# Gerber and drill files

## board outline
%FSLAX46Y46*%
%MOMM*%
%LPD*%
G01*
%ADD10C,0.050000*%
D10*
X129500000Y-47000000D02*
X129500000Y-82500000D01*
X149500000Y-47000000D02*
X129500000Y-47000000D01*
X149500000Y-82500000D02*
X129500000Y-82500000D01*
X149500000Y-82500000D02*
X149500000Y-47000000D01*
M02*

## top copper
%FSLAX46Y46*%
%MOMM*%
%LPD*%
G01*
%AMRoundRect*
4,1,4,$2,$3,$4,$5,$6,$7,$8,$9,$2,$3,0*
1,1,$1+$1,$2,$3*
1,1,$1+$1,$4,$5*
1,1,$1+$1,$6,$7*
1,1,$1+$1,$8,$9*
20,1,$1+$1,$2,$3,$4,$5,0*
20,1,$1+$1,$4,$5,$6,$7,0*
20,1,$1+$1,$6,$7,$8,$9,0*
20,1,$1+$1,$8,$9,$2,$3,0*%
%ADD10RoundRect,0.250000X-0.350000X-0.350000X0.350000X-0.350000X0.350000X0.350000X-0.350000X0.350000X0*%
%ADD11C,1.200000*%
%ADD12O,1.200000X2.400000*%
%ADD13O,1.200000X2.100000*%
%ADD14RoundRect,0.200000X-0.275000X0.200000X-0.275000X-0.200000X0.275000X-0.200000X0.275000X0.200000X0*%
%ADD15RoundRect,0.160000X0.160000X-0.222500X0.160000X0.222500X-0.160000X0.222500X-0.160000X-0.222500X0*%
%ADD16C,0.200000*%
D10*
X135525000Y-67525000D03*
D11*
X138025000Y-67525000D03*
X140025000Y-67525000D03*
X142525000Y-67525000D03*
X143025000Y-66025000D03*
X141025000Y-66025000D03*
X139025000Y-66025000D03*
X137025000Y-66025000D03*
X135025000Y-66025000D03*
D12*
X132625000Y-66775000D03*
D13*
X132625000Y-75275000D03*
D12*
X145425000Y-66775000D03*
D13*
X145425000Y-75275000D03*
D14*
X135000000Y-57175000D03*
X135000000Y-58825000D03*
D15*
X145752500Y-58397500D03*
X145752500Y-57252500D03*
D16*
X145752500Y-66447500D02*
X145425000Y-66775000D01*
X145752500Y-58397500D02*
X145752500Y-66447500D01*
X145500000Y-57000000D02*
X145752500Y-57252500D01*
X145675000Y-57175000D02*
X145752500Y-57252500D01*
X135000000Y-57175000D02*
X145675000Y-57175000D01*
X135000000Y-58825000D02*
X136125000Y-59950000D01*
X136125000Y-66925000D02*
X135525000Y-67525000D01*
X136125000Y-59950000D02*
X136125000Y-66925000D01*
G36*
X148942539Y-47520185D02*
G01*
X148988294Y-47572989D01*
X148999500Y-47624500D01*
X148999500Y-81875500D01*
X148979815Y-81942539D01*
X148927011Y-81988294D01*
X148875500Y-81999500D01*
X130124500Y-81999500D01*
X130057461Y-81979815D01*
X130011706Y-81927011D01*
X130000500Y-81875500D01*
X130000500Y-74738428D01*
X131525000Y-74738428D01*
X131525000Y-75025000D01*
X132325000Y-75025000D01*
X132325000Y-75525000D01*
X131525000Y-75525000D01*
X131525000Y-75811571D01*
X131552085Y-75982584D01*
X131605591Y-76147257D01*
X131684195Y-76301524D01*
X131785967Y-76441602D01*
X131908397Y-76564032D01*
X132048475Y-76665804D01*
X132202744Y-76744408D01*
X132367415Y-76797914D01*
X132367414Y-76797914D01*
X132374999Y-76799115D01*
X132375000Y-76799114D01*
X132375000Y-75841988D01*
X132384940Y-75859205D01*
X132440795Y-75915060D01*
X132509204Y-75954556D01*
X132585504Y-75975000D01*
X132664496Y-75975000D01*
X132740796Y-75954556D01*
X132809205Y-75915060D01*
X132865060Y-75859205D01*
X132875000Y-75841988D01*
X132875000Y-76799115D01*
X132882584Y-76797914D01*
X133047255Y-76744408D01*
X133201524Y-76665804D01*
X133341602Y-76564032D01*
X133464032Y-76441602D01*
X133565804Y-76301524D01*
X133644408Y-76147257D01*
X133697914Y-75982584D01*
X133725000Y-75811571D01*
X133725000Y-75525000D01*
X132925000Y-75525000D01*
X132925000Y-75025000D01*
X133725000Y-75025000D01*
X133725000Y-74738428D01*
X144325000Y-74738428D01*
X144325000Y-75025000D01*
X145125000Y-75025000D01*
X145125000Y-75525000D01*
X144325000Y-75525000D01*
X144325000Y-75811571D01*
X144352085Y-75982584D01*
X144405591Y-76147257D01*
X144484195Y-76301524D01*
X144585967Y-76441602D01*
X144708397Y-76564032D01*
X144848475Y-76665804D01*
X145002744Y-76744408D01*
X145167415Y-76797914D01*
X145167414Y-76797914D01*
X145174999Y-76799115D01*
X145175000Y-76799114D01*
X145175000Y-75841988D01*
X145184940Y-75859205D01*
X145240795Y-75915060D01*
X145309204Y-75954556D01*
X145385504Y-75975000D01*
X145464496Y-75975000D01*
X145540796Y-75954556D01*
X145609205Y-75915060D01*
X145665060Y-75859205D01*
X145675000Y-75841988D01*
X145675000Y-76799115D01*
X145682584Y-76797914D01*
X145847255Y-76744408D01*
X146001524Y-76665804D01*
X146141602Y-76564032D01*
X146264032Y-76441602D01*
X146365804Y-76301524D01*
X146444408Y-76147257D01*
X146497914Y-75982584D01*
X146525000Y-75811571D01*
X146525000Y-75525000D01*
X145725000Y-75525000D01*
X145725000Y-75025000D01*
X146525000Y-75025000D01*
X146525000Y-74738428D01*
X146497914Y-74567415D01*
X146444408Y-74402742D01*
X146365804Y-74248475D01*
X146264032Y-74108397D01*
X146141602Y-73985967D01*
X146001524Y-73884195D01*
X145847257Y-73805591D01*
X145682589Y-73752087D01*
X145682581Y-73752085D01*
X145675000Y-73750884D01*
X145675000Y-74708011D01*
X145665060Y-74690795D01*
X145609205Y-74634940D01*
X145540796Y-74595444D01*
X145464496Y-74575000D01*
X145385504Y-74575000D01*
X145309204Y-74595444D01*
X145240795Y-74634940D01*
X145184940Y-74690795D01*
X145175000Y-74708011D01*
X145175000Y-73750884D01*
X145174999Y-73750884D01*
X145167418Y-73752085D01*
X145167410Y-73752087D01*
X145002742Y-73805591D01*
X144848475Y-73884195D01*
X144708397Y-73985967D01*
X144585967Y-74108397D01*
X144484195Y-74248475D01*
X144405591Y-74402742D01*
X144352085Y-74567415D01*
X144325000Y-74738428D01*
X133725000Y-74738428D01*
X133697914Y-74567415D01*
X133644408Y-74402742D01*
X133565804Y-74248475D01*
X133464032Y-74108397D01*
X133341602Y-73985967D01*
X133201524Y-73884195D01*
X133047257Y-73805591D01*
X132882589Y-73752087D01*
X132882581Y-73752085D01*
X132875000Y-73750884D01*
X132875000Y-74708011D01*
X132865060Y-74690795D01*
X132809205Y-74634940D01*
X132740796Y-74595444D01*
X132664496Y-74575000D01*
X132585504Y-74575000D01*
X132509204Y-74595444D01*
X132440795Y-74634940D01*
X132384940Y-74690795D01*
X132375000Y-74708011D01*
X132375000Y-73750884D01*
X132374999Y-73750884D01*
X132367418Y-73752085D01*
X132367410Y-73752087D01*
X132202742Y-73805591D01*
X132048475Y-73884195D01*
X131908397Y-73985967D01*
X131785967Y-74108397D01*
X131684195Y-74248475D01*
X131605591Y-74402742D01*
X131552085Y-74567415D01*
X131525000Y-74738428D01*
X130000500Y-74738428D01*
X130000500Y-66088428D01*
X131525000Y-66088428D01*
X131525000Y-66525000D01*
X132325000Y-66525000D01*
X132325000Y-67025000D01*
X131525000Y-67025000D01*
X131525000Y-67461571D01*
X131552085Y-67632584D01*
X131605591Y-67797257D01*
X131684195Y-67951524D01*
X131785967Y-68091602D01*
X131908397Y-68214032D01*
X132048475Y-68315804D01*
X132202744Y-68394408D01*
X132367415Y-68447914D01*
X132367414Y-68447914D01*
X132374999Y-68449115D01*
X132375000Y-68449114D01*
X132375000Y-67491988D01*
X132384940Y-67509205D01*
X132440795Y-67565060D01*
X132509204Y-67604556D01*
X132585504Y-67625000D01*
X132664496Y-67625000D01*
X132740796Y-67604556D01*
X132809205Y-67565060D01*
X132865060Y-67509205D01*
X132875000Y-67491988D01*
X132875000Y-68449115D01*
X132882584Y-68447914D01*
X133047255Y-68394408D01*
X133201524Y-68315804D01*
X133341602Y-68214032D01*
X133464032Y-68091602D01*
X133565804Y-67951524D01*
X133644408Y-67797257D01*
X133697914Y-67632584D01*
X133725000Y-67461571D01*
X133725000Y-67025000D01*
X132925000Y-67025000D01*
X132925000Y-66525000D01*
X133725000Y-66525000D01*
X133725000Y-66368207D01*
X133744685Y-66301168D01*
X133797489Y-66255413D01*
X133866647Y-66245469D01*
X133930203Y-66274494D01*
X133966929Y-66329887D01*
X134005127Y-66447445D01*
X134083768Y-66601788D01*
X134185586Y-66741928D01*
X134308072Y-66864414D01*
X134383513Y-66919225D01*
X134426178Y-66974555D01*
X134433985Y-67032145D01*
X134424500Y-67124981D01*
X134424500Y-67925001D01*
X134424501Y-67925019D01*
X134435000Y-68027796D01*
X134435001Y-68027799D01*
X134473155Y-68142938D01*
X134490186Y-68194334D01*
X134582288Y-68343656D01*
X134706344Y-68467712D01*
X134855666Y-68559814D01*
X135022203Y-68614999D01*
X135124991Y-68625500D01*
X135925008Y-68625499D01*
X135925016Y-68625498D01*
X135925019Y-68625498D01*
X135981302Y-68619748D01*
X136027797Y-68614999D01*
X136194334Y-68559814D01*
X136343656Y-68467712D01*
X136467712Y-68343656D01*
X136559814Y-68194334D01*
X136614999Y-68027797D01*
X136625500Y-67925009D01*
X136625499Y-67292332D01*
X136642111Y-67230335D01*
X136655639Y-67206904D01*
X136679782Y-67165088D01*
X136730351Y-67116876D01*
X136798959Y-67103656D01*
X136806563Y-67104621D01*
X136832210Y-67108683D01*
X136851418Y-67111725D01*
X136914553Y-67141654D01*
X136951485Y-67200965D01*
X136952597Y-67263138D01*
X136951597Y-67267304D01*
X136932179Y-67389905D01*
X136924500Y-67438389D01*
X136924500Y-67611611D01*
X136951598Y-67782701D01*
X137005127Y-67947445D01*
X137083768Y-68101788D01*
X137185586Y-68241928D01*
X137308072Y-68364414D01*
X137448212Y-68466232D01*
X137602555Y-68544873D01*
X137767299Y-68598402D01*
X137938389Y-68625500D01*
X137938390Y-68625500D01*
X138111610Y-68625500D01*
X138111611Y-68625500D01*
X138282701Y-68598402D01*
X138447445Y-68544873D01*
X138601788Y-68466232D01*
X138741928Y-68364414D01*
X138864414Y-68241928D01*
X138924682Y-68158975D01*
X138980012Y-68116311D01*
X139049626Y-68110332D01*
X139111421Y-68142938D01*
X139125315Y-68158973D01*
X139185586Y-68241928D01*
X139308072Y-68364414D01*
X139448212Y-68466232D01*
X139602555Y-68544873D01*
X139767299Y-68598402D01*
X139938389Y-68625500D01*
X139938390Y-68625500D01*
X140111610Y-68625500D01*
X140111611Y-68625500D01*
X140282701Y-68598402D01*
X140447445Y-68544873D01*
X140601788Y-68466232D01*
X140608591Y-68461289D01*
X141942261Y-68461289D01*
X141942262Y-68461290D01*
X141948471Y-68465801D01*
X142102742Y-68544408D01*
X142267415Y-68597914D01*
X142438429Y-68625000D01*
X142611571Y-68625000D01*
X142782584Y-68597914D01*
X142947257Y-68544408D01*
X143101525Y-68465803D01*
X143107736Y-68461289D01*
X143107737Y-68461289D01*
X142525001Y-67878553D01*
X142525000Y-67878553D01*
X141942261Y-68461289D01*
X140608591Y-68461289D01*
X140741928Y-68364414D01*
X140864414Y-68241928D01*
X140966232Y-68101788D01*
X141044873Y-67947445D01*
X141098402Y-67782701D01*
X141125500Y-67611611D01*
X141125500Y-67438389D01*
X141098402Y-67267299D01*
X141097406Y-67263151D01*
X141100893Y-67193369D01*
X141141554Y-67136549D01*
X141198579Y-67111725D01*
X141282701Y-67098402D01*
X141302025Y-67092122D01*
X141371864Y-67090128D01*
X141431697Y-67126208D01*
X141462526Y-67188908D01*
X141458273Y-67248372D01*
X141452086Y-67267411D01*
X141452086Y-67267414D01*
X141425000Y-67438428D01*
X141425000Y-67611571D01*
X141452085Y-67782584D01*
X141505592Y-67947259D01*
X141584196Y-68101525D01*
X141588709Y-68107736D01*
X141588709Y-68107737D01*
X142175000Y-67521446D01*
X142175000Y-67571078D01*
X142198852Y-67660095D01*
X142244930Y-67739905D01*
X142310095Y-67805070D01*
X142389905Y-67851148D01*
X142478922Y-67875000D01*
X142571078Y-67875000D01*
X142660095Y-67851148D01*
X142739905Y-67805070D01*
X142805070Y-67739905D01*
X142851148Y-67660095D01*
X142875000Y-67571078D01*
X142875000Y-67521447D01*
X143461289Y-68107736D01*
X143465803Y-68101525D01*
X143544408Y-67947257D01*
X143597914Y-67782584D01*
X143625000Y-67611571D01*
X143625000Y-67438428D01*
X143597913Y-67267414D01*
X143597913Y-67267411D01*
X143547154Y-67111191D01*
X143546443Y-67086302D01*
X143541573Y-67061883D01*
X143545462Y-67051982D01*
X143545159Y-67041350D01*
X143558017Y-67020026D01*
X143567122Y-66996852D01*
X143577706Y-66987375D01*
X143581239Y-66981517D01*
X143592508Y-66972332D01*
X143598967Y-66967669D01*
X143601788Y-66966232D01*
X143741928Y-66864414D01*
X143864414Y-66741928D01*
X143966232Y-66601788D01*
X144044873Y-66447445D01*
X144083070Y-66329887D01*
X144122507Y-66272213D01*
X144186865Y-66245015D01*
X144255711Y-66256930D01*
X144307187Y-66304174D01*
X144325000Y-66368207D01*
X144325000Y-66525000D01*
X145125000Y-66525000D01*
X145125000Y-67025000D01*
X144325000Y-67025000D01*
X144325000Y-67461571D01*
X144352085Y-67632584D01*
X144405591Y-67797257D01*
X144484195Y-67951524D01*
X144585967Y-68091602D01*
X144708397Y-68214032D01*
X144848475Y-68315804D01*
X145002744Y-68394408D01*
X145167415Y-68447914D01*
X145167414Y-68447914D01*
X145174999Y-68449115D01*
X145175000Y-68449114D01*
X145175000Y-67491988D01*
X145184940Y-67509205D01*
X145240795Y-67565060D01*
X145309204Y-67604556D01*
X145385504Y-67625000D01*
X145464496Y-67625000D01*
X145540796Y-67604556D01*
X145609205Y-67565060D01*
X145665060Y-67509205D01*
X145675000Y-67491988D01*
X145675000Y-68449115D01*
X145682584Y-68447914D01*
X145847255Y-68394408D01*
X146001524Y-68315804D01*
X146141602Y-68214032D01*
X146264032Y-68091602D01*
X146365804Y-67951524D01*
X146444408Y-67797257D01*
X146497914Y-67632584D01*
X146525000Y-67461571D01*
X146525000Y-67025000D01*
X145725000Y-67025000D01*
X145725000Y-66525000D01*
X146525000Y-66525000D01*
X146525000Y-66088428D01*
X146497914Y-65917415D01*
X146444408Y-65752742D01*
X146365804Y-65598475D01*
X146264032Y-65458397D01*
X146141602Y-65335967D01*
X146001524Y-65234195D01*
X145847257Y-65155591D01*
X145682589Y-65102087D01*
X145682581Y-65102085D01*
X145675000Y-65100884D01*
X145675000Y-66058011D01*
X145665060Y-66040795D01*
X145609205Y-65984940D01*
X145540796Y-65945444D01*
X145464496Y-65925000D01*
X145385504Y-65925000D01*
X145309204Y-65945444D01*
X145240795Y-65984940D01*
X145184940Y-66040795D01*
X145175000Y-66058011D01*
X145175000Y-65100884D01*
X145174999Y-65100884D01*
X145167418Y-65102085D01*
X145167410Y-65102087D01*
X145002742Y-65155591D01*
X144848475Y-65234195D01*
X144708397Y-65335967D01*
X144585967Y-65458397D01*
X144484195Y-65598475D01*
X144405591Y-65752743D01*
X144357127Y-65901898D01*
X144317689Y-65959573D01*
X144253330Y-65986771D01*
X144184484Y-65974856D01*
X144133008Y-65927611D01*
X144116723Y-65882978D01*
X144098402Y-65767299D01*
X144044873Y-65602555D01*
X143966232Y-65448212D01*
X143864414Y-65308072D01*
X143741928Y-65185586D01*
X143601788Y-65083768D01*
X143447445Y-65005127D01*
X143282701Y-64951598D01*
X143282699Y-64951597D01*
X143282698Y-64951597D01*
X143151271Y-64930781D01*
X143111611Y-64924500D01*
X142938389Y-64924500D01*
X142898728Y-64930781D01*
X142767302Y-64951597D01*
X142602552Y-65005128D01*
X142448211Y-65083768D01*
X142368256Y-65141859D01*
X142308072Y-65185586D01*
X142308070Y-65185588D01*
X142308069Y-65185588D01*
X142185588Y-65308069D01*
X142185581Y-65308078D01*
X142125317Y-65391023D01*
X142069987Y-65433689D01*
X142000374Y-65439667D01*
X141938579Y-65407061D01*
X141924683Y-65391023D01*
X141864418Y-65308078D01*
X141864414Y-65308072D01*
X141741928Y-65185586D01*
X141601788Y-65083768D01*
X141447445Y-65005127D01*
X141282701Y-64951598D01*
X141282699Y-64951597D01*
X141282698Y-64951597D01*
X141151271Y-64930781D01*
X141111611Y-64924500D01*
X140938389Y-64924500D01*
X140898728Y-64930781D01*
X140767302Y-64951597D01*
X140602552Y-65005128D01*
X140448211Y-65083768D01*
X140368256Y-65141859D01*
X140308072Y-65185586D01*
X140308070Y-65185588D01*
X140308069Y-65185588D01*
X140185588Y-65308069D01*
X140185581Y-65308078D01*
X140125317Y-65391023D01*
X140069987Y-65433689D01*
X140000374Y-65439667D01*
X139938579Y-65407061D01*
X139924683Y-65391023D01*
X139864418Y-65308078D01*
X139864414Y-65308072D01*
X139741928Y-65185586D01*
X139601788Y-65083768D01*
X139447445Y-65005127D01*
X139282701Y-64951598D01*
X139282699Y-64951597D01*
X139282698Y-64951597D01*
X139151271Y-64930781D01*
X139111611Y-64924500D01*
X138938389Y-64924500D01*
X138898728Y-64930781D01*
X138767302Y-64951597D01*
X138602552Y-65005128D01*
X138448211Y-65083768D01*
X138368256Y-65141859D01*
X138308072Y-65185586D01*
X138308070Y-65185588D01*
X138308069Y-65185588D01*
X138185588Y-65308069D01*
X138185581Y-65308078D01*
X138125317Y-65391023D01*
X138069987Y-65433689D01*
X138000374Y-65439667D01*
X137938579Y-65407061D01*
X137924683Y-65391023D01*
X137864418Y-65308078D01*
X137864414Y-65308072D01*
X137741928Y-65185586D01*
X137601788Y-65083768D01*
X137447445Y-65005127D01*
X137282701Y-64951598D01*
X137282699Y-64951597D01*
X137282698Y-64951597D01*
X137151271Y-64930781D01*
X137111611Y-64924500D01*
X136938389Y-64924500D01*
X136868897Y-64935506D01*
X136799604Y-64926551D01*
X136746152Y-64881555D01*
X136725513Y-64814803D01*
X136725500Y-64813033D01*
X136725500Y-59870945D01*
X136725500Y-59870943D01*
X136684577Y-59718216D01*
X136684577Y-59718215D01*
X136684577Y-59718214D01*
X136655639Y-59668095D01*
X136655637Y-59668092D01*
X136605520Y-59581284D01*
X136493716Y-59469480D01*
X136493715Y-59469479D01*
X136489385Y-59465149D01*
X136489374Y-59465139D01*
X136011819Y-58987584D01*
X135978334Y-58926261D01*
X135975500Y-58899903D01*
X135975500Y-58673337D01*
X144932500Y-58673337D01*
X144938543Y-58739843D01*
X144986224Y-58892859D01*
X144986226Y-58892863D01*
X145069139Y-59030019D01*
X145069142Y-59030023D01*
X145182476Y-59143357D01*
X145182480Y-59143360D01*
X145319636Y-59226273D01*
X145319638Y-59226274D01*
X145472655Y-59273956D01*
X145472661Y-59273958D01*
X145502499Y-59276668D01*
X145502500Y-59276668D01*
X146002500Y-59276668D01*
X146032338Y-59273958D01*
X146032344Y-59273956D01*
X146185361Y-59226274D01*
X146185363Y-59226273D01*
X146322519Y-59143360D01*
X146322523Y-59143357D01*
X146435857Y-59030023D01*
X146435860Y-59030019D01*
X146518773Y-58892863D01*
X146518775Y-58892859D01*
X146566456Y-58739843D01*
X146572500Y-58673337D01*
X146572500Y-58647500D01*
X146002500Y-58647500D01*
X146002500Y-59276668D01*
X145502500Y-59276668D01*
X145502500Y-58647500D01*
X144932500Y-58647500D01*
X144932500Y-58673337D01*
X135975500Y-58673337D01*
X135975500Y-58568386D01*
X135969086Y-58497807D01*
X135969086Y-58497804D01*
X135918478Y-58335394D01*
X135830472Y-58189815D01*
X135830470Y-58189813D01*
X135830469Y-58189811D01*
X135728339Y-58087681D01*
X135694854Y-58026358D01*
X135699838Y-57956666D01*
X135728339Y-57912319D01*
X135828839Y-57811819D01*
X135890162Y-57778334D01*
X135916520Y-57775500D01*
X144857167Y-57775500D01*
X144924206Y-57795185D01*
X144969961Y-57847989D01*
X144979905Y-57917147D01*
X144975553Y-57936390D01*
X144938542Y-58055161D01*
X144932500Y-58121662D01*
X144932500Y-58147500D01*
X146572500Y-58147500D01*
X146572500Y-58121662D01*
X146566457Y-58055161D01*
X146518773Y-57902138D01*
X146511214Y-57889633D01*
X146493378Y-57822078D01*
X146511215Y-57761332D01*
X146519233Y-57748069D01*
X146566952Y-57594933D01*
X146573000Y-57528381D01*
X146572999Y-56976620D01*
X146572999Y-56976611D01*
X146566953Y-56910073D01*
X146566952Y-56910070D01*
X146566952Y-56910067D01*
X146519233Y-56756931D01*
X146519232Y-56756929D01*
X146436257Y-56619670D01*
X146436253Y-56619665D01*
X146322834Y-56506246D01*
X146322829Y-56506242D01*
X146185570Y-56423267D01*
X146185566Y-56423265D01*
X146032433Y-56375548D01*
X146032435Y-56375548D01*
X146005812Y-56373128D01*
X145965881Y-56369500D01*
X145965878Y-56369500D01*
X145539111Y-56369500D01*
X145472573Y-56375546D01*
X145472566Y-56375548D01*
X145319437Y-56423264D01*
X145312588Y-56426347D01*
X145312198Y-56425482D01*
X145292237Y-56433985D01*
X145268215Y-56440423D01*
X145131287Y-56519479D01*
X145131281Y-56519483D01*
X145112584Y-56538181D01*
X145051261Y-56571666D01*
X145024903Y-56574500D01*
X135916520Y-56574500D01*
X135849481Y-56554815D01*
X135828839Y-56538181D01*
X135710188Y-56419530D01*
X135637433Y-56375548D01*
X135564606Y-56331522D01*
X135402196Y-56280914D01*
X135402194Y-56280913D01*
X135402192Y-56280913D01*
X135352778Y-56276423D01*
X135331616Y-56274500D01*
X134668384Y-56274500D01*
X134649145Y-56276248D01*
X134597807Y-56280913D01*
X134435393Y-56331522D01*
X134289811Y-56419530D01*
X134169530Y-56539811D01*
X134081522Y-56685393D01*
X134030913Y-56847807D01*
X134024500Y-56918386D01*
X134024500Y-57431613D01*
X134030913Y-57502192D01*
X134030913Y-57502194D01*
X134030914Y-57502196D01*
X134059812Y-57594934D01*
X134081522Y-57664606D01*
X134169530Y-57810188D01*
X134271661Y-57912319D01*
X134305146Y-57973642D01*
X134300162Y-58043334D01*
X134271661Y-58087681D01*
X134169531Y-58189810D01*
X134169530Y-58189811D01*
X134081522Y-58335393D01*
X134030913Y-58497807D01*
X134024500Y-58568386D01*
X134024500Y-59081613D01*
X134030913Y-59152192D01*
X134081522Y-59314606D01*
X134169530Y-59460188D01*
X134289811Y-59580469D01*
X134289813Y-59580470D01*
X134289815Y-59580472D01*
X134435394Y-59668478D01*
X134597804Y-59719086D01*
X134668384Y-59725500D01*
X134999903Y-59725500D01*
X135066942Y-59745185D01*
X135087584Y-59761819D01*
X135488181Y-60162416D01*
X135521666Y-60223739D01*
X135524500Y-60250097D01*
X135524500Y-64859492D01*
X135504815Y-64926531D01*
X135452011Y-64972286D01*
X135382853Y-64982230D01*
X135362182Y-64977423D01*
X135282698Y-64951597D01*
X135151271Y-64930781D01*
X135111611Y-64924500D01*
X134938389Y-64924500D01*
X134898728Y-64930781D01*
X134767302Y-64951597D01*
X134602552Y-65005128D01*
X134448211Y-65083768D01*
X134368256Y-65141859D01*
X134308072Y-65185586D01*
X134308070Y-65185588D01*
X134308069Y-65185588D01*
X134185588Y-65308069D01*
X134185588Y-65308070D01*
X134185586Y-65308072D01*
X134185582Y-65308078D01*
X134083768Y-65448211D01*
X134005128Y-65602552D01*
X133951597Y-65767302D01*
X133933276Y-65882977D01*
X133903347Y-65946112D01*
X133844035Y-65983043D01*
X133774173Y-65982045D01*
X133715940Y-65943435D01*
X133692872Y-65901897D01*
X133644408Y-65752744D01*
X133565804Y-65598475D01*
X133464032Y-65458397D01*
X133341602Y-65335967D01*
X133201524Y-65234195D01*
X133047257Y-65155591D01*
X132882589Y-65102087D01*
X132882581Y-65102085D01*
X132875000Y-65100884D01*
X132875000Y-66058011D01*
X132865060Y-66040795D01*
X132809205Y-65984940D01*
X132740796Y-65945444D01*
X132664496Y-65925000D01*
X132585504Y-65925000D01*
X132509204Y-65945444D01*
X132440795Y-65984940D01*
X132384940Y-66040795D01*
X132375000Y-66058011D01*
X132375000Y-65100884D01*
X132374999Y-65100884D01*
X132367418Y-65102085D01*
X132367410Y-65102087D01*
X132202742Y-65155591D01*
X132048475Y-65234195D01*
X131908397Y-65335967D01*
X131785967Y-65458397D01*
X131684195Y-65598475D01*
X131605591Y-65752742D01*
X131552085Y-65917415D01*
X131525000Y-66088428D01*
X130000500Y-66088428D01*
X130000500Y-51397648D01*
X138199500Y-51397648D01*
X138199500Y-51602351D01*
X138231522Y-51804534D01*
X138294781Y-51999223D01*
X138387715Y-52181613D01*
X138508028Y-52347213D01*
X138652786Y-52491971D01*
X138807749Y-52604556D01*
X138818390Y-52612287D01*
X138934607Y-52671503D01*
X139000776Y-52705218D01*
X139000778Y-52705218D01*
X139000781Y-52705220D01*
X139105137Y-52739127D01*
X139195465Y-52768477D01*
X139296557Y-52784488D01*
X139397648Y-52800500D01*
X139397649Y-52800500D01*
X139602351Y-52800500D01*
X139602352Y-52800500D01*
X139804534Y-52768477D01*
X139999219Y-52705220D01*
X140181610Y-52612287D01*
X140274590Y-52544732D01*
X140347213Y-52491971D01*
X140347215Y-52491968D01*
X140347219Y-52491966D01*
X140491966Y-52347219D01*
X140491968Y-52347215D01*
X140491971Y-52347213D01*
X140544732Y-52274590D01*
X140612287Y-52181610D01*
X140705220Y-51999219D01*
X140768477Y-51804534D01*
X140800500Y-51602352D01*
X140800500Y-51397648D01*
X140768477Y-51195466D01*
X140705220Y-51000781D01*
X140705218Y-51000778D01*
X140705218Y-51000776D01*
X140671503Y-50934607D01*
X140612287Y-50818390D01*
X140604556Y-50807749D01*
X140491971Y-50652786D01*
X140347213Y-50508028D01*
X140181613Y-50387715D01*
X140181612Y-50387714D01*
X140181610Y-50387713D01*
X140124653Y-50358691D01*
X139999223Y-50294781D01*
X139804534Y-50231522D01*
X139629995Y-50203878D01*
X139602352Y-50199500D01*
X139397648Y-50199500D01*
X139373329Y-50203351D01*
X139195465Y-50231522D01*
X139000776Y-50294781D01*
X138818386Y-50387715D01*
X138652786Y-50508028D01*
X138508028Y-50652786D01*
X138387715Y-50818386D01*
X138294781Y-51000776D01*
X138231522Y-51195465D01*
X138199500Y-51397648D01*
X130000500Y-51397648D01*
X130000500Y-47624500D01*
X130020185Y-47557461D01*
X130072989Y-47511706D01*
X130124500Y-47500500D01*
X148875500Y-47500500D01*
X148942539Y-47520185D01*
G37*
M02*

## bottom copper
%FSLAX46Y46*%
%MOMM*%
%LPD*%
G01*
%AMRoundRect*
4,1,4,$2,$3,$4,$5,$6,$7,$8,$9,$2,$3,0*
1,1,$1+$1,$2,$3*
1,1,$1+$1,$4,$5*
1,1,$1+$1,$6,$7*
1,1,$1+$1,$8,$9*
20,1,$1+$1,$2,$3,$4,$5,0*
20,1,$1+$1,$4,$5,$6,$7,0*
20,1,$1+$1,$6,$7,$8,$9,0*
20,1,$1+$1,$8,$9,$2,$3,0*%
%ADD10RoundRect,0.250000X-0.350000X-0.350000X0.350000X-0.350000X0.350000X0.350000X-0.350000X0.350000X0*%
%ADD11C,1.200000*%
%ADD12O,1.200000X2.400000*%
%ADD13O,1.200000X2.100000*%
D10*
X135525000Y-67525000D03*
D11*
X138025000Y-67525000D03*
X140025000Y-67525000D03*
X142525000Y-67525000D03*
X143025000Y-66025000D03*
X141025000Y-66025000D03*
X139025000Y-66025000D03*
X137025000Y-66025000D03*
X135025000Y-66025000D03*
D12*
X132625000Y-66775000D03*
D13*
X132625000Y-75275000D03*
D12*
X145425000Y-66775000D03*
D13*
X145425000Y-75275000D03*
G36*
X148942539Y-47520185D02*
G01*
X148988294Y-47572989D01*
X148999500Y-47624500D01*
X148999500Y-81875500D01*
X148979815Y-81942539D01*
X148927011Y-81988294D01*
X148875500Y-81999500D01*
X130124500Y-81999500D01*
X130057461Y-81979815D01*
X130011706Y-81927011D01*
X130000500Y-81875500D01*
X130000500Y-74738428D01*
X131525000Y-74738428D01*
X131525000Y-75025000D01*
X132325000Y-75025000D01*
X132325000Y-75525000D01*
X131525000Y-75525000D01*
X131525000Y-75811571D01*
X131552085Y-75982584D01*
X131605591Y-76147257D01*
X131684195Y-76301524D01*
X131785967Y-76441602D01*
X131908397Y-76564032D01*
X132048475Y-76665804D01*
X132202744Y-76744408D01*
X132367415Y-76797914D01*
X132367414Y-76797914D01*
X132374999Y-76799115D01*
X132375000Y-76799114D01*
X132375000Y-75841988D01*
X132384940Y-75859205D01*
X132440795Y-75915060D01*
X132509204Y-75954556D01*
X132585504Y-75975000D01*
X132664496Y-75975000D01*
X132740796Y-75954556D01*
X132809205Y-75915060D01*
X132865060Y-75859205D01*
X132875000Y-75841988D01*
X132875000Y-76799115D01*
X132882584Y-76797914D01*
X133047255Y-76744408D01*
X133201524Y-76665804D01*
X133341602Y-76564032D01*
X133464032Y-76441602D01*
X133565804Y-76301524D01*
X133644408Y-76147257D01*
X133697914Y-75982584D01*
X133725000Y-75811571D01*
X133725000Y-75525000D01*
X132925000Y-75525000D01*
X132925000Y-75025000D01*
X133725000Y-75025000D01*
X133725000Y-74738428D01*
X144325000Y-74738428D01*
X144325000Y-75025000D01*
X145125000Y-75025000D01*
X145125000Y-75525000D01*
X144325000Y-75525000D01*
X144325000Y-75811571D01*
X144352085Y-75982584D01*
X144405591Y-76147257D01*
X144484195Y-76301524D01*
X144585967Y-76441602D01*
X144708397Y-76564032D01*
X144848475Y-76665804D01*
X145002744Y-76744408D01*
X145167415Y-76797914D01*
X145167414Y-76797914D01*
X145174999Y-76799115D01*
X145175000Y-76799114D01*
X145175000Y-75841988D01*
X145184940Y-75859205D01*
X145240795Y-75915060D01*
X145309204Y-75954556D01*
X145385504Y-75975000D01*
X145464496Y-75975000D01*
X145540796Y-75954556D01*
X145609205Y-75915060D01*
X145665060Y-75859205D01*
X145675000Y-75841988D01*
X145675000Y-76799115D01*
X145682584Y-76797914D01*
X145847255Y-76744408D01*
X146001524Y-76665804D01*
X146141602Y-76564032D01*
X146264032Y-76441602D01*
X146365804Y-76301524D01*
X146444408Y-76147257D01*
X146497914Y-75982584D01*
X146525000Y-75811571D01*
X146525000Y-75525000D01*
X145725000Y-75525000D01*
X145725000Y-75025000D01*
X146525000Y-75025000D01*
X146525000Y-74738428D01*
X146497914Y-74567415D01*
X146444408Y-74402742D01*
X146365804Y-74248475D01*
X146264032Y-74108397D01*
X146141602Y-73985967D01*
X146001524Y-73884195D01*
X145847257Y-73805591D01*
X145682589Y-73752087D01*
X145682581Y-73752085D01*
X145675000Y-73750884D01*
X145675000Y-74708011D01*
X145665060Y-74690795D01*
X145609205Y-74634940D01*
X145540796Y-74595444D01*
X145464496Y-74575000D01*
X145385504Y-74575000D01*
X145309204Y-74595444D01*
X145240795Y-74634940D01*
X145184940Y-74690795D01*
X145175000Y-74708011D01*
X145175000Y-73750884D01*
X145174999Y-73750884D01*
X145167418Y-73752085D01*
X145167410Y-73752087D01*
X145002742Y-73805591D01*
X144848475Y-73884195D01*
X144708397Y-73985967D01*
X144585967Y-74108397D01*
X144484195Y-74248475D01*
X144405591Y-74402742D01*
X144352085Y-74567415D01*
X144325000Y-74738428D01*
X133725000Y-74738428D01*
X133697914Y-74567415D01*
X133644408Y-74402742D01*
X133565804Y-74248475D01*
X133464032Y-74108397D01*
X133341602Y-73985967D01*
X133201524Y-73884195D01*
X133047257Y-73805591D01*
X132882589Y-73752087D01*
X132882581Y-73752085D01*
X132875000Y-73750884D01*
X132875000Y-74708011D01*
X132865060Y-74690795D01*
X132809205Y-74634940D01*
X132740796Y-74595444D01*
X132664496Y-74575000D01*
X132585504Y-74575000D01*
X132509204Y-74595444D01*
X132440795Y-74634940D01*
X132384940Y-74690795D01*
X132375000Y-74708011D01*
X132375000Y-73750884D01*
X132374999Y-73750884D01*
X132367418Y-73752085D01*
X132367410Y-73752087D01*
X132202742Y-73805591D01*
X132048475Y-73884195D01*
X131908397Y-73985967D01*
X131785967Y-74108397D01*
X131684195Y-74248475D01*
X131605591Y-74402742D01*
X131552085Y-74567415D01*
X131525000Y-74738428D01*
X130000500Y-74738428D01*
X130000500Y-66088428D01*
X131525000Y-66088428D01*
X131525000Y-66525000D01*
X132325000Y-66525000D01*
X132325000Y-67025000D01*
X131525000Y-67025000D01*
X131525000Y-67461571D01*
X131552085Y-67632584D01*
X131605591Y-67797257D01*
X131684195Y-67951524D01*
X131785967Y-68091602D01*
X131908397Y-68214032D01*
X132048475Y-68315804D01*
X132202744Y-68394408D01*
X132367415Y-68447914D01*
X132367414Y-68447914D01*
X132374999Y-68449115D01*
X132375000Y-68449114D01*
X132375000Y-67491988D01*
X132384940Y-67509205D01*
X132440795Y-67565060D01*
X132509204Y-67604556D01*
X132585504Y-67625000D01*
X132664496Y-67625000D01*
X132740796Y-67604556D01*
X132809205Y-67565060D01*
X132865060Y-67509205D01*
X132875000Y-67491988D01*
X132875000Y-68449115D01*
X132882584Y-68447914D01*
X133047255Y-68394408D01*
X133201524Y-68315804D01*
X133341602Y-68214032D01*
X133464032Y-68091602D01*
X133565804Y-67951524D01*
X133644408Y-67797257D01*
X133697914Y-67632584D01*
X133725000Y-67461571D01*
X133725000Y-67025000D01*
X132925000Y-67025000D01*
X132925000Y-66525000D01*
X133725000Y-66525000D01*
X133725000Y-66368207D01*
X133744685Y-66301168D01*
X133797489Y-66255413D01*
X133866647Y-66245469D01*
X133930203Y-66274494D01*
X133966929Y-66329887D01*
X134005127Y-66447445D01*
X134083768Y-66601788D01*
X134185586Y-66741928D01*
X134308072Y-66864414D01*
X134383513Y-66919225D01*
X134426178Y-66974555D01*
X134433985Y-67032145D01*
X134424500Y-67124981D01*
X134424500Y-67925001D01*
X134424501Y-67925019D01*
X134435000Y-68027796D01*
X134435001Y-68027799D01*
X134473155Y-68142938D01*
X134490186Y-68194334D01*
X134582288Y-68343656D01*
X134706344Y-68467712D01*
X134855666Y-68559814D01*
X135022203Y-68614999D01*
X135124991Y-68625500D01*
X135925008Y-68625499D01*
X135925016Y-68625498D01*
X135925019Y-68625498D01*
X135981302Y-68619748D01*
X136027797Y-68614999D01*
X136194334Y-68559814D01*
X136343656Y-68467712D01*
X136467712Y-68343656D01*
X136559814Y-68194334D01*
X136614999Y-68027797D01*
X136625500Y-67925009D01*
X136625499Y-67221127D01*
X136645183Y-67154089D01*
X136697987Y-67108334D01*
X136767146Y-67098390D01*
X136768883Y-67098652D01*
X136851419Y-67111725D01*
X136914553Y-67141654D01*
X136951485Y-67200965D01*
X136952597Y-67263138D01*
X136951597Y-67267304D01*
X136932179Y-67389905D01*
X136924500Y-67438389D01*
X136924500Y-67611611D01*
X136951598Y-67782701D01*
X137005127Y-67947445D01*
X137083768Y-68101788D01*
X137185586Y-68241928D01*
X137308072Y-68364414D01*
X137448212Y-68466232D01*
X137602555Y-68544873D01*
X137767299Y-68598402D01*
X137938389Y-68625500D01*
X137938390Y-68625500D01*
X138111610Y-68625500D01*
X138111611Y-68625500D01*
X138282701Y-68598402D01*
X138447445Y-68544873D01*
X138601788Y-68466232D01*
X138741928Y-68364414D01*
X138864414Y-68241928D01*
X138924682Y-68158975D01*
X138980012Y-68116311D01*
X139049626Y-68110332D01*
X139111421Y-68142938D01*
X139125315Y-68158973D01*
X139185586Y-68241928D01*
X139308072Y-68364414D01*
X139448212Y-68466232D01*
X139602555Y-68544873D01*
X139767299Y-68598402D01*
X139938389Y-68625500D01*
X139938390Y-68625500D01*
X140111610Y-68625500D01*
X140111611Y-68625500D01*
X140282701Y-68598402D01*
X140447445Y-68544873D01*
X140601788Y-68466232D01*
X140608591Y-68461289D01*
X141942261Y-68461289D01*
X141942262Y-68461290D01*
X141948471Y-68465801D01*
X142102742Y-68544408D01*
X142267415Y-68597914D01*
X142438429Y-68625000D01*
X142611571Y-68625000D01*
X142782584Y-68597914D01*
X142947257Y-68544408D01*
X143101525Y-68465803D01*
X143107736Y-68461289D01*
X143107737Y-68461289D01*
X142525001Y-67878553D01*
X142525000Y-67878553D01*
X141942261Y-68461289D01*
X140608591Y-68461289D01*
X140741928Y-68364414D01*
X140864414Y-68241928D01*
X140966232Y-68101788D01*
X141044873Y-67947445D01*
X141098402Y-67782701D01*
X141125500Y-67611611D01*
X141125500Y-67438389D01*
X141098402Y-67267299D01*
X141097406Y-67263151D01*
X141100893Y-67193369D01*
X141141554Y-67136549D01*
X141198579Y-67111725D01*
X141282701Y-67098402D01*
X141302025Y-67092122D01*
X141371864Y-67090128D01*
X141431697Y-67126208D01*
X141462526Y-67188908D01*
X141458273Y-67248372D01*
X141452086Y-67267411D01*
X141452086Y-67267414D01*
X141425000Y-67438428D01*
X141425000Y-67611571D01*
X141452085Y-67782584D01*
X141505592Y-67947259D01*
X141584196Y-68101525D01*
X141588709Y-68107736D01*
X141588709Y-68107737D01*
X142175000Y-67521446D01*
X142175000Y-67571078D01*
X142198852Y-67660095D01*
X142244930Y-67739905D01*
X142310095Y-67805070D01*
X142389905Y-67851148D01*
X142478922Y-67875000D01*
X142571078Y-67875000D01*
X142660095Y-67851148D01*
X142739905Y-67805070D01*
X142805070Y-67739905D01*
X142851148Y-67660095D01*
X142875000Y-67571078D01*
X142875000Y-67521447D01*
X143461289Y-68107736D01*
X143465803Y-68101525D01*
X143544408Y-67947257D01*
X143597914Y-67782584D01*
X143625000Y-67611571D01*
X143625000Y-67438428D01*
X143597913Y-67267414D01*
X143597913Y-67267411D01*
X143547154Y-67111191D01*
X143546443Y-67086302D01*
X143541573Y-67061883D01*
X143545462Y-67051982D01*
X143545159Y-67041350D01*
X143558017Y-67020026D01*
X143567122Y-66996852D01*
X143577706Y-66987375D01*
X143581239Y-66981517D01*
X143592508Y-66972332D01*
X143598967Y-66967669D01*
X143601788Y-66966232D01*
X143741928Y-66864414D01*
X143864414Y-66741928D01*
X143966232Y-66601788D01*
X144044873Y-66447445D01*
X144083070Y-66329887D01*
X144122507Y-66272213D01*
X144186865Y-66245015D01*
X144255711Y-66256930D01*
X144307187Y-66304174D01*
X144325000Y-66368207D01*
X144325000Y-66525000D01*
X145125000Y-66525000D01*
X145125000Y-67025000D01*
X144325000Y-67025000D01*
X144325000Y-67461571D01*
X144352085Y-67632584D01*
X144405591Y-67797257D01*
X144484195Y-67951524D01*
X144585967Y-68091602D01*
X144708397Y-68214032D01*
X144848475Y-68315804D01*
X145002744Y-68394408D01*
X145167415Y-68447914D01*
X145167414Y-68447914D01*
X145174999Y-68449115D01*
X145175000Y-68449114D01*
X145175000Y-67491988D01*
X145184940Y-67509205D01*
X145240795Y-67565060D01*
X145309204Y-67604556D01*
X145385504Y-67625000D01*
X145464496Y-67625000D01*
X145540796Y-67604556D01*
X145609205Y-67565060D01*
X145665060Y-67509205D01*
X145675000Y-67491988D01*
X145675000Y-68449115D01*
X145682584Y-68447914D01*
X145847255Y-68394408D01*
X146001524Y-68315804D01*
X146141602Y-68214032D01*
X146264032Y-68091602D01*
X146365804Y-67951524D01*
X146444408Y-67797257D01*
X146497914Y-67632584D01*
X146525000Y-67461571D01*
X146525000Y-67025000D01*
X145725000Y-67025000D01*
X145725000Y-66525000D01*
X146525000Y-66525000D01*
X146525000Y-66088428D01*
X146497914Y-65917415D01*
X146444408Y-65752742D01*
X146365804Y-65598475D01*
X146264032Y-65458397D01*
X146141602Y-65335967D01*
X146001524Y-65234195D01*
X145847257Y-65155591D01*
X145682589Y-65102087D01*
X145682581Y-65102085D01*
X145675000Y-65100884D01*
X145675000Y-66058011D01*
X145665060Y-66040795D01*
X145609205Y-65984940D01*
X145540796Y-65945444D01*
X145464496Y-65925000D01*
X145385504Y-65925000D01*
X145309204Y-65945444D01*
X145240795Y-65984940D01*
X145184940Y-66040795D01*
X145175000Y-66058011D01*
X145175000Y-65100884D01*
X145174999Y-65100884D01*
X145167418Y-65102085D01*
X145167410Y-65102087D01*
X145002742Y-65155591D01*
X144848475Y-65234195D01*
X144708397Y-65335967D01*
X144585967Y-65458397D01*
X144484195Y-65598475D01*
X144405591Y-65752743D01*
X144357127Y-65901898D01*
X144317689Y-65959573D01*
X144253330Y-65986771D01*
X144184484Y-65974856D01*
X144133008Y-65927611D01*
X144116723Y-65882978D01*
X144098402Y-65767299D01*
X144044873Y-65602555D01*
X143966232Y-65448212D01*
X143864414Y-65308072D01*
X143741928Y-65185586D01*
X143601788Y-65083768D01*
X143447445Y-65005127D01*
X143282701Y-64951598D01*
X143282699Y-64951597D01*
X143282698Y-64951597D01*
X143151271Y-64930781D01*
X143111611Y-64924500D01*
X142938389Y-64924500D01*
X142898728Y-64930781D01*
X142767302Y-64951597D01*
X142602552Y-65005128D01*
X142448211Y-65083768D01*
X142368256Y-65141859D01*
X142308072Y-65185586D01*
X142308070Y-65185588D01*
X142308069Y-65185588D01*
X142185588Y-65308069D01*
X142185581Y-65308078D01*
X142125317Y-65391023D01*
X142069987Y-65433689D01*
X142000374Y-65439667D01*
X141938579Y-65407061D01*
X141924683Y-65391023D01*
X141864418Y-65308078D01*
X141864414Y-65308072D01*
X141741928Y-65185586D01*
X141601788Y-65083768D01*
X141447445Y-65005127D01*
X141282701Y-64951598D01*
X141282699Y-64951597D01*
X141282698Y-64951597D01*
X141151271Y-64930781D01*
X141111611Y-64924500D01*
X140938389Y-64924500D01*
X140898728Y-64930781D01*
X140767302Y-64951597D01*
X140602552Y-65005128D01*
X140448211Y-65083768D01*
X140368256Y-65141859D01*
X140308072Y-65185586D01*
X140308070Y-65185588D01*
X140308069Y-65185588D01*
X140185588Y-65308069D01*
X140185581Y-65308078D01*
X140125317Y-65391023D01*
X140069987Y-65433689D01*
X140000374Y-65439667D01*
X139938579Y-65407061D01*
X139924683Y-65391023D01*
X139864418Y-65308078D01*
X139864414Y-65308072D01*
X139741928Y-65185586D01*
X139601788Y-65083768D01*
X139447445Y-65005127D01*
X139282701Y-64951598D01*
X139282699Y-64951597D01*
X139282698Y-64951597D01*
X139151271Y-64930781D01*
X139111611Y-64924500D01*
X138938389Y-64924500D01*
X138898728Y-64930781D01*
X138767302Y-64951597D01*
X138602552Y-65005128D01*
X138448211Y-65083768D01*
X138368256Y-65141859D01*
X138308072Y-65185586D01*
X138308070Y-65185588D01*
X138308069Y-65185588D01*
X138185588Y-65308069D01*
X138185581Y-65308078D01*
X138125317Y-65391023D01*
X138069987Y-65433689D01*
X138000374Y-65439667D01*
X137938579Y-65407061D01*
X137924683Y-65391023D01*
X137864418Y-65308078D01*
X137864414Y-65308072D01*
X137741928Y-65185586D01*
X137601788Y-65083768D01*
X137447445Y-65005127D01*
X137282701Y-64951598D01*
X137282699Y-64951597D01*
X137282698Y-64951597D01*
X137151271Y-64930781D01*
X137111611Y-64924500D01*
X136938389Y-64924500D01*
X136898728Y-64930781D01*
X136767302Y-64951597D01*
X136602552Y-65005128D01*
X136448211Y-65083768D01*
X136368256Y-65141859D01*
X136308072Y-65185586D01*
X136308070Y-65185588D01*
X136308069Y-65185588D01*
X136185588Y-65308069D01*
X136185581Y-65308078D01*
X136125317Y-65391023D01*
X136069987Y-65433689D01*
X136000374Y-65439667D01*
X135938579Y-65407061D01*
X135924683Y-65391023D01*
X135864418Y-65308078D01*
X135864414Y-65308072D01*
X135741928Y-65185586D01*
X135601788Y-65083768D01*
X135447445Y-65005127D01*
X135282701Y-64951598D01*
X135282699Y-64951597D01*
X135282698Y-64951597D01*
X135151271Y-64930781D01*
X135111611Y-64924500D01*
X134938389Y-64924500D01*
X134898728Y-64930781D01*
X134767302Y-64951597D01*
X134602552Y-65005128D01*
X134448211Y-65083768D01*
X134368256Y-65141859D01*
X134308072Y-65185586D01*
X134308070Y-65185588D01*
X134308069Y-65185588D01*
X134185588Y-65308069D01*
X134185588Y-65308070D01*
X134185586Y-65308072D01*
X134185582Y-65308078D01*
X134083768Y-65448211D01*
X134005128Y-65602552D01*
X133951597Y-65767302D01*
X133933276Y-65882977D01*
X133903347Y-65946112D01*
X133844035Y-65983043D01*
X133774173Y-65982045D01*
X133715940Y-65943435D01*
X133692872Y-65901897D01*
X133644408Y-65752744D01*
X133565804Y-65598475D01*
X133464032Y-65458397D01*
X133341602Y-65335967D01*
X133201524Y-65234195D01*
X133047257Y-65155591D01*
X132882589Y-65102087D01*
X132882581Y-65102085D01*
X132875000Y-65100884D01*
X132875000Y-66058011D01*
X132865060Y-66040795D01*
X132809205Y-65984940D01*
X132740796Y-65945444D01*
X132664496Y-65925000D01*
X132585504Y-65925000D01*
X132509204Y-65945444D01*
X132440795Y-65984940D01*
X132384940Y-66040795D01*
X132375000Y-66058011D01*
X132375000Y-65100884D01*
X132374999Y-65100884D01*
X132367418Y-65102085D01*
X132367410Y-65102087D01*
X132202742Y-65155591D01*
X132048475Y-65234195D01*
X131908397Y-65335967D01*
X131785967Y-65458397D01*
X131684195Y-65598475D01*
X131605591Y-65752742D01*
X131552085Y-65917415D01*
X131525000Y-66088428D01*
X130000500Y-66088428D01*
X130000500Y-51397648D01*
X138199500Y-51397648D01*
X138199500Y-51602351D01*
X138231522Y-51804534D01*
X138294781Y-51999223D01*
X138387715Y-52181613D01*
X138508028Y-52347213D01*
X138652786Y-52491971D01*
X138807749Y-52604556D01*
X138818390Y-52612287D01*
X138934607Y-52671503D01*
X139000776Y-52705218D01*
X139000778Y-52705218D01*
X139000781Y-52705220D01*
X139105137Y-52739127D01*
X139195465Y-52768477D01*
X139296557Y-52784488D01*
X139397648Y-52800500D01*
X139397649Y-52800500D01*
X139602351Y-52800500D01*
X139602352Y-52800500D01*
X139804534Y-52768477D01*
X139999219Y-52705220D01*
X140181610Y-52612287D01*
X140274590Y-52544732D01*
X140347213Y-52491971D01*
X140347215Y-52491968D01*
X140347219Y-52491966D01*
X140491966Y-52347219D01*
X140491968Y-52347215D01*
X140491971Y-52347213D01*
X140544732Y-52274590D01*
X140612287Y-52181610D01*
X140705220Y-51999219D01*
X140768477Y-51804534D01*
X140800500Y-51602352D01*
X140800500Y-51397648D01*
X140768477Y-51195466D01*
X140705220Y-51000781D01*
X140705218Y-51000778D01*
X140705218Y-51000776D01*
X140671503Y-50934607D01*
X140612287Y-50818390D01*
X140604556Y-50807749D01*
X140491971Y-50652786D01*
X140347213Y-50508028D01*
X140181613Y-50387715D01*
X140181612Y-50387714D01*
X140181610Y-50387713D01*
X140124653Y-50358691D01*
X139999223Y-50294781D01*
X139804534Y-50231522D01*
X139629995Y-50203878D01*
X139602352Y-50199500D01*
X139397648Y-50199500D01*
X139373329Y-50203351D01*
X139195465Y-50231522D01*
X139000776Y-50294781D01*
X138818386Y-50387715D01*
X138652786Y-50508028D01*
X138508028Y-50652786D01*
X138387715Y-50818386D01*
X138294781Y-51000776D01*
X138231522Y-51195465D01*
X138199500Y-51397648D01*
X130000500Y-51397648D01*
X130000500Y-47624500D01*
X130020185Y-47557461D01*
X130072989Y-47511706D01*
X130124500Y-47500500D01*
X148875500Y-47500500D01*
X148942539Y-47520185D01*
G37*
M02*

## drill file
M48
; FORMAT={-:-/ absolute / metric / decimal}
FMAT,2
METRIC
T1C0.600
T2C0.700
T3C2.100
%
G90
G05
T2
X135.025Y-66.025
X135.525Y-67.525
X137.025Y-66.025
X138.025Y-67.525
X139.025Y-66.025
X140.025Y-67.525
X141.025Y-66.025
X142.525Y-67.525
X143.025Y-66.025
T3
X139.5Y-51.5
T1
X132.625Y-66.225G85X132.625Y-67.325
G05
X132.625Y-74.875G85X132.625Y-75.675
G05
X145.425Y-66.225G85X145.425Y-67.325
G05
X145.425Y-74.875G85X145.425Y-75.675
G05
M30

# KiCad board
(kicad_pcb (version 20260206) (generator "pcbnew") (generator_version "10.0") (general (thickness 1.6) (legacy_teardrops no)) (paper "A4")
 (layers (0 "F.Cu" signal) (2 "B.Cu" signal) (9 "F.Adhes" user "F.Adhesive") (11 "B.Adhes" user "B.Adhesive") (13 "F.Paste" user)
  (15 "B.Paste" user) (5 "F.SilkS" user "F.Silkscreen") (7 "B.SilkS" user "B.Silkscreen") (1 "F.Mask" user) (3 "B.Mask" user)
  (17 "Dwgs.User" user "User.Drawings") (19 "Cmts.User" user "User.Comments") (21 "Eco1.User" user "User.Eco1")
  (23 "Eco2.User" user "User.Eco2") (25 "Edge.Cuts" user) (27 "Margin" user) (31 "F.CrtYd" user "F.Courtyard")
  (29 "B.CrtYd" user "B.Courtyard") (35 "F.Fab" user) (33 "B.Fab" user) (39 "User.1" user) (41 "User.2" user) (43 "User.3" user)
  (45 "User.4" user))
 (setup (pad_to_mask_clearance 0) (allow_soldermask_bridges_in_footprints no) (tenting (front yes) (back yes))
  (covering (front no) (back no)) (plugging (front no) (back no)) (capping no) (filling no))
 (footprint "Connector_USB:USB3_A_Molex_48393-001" (layer "F.Cu") (at 135.525 67.525)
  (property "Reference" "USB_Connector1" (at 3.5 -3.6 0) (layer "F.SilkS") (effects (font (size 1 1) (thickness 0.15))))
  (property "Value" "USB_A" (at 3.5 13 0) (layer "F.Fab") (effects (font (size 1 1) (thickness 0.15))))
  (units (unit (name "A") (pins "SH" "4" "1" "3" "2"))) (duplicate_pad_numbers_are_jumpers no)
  (pad "1" thru_hole roundrect (at 0 0) (size 1.2 1.2) (drill 0.7) (layers "*.Cu" "*.Mask") (remove_unused_layers no)
   (roundrect_rratio 0.2083333333) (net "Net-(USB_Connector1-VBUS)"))
  (pad "2" thru_hole circle (at 2.5 0) (size 1.2 1.2) (drill 0.7) (layers "*.Cu" "*.Mask") (remove_unused_layers no)
   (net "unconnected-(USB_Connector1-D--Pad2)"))
  (pad "3" thru_hole circle (at 4.5 0) (size 1.2 1.2) (drill 0.7) (layers "*.Cu" "*.Mask") (remove_unused_layers no)
   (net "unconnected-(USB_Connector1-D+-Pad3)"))
  (pad "4" thru_hole circle (at 7 0) (size 1.2 1.2) (drill 0.7) (layers "*.Cu" "*.Mask") (remove_unused_layers no) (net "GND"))
  (pad "5" thru_hole circle (at 7.5 -1.5) (size 1.2 1.2) (drill 0.7) (layers "*.Cu" "*.Mask") (remove_unused_layers no))
  (pad "6" thru_hole circle (at 5.5 -1.5) (size 1.2 1.2) (drill 0.7) (layers "*.Cu" "*.Mask") (remove_unused_layers no))
  (pad "7" thru_hole circle (at 3.5 -1.5) (size 1.2 1.2) (drill 0.7) (layers "*.Cu" "*.Mask") (remove_unused_layers no))
  (pad "8" thru_hole circle (at 1.5 -1.5) (size 1.2 1.2) (drill 0.7) (layers "*.Cu" "*.Mask") (remove_unused_layers no))
  (pad "9" thru_hole circle (at -0.5 -1.5) (size 1.2 1.2) (drill 0.7) (layers "*.Cu" "*.Mask") (remove_unused_layers no))
  (pad "SH" thru_hole oval (at -2.9 -0.75) (size 1.2 2.4) (drill oval 0.6 1.7) (layers "*.Cu" "*.Mask") (remove_unused_layers no)
   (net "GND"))
  (pad "SH" thru_hole oval (at -2.9 7.75) (size 1.2 2.1) (drill oval 0.6 1.4) (layers "*.Cu" "*.Mask") (remove_unused_layers no) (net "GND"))
  (pad "SH" thru_hole oval (at 9.9 -0.75) (size 1.2 2.4) (drill oval 0.6 1.7) (layers "*.Cu" "*.Mask") (remove_unused_layers no) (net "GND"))
  (pad "SH" thru_hole oval (at 9.9 7.75) (size 1.2 2.1) (drill oval 0.6 1.4) (layers "*.Cu" "*.Mask") (remove_unused_layers no) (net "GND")))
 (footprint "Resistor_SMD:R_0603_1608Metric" (layer "F.Cu") (at 135 58 -90)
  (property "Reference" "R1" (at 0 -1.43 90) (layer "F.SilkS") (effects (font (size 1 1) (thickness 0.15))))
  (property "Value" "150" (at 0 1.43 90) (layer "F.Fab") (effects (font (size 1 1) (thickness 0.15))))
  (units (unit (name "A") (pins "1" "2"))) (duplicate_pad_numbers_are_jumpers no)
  (pad "1" smd roundrect (at -0.825 0 270) (size 0.8 0.95) (layers "F.Cu" "F.Mask" "F.Paste") (roundrect_rratio 0.25) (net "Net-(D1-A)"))
  (pad "2" smd roundrect (at 0.825 0 270) (size 0.8 0.95) (layers "F.Cu" "F.Mask" "F.Paste") (roundrect_rratio 0.25)
   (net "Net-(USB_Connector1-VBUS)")))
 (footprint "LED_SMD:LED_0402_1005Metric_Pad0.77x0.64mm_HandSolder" (layer "F.Cu") (at 145.7525 57.825 90)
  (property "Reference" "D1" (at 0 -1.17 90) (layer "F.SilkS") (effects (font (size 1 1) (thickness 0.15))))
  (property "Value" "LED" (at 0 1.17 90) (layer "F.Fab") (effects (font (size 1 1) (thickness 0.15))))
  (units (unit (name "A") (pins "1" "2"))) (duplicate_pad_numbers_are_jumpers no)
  (pad "1" smd roundrect (at -0.5725 0 90) (size 0.765 0.64) (layers "F.Cu" "F.Mask" "F.Paste") (roundrect_rratio 0.25) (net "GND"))
  (pad "2" smd roundrect (at 0.5725 0 90) (size 0.765 0.64) (layers "F.Cu" "F.Mask" "F.Paste") (roundrect_rratio 0.25) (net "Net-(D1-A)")))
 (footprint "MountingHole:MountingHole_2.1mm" (layer "F.Cu") (at 139.5 51.5)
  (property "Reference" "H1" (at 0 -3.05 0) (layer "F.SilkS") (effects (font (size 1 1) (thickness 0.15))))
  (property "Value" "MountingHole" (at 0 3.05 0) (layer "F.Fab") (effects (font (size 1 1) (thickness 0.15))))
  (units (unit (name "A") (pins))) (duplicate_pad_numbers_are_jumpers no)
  (pad "" np_thru_hole circle (at 0 0) (size 2.1 2.1) (drill 2.1) (layers "*.Cu" "*.Mask")))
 (gr_line (start 129.5 47) (end 129.5 82.5) (stroke (width 0.05) (type default)) (layer "Edge.Cuts"))
 (gr_line (start 149.5 47) (end 129.5 47) (stroke (width 0.05) (type default)) (layer "Edge.Cuts"))
 (gr_line (start 149.5 82.5) (end 129.5 82.5) (stroke (width 0.05) (type default)) (layer "Edge.Cuts"))
 (gr_line (start 149.5 82.5) (end 149.5 47) (stroke (width 0.05) (type default)) (layer "Edge.Cuts"))
 (segment (start 145.7525 66.4475) (end 145.425 66.775) (width 0.2) (layer "F.Cu") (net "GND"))
 (segment (start 145.7525 58.3975) (end 145.7525 66.4475) (width 0.2) (layer "F.Cu") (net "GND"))
 (segment (start 145.5 57) (end 145.7525 57.2525) (width 0.2) (layer "F.Cu") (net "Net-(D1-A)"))
 (segment (start 145.675 57.175) (end 145.7525 57.2525) (width 0.2) (layer "F.Cu") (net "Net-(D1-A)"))
 (segment (start 135 57.175) (end 145.675 57.175) (width 0.2) (layer "F.Cu") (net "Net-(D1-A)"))
 (segment (start 135 58.825) (end 136.125 59.95) (width 0.2) (layer "F.Cu") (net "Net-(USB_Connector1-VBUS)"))
 (segment (start 136.125 66.925) (end 135.525 67.525) (width 0.2) (layer "F.Cu") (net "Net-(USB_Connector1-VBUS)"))
 (segment (start 136.125 59.95) (end 136.125 66.925) (width 0.2) (layer "F.Cu") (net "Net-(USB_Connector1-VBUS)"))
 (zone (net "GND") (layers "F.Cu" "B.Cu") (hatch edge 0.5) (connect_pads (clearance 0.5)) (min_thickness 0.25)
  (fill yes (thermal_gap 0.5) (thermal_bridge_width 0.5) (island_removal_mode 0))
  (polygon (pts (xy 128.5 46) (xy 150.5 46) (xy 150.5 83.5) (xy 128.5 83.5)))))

